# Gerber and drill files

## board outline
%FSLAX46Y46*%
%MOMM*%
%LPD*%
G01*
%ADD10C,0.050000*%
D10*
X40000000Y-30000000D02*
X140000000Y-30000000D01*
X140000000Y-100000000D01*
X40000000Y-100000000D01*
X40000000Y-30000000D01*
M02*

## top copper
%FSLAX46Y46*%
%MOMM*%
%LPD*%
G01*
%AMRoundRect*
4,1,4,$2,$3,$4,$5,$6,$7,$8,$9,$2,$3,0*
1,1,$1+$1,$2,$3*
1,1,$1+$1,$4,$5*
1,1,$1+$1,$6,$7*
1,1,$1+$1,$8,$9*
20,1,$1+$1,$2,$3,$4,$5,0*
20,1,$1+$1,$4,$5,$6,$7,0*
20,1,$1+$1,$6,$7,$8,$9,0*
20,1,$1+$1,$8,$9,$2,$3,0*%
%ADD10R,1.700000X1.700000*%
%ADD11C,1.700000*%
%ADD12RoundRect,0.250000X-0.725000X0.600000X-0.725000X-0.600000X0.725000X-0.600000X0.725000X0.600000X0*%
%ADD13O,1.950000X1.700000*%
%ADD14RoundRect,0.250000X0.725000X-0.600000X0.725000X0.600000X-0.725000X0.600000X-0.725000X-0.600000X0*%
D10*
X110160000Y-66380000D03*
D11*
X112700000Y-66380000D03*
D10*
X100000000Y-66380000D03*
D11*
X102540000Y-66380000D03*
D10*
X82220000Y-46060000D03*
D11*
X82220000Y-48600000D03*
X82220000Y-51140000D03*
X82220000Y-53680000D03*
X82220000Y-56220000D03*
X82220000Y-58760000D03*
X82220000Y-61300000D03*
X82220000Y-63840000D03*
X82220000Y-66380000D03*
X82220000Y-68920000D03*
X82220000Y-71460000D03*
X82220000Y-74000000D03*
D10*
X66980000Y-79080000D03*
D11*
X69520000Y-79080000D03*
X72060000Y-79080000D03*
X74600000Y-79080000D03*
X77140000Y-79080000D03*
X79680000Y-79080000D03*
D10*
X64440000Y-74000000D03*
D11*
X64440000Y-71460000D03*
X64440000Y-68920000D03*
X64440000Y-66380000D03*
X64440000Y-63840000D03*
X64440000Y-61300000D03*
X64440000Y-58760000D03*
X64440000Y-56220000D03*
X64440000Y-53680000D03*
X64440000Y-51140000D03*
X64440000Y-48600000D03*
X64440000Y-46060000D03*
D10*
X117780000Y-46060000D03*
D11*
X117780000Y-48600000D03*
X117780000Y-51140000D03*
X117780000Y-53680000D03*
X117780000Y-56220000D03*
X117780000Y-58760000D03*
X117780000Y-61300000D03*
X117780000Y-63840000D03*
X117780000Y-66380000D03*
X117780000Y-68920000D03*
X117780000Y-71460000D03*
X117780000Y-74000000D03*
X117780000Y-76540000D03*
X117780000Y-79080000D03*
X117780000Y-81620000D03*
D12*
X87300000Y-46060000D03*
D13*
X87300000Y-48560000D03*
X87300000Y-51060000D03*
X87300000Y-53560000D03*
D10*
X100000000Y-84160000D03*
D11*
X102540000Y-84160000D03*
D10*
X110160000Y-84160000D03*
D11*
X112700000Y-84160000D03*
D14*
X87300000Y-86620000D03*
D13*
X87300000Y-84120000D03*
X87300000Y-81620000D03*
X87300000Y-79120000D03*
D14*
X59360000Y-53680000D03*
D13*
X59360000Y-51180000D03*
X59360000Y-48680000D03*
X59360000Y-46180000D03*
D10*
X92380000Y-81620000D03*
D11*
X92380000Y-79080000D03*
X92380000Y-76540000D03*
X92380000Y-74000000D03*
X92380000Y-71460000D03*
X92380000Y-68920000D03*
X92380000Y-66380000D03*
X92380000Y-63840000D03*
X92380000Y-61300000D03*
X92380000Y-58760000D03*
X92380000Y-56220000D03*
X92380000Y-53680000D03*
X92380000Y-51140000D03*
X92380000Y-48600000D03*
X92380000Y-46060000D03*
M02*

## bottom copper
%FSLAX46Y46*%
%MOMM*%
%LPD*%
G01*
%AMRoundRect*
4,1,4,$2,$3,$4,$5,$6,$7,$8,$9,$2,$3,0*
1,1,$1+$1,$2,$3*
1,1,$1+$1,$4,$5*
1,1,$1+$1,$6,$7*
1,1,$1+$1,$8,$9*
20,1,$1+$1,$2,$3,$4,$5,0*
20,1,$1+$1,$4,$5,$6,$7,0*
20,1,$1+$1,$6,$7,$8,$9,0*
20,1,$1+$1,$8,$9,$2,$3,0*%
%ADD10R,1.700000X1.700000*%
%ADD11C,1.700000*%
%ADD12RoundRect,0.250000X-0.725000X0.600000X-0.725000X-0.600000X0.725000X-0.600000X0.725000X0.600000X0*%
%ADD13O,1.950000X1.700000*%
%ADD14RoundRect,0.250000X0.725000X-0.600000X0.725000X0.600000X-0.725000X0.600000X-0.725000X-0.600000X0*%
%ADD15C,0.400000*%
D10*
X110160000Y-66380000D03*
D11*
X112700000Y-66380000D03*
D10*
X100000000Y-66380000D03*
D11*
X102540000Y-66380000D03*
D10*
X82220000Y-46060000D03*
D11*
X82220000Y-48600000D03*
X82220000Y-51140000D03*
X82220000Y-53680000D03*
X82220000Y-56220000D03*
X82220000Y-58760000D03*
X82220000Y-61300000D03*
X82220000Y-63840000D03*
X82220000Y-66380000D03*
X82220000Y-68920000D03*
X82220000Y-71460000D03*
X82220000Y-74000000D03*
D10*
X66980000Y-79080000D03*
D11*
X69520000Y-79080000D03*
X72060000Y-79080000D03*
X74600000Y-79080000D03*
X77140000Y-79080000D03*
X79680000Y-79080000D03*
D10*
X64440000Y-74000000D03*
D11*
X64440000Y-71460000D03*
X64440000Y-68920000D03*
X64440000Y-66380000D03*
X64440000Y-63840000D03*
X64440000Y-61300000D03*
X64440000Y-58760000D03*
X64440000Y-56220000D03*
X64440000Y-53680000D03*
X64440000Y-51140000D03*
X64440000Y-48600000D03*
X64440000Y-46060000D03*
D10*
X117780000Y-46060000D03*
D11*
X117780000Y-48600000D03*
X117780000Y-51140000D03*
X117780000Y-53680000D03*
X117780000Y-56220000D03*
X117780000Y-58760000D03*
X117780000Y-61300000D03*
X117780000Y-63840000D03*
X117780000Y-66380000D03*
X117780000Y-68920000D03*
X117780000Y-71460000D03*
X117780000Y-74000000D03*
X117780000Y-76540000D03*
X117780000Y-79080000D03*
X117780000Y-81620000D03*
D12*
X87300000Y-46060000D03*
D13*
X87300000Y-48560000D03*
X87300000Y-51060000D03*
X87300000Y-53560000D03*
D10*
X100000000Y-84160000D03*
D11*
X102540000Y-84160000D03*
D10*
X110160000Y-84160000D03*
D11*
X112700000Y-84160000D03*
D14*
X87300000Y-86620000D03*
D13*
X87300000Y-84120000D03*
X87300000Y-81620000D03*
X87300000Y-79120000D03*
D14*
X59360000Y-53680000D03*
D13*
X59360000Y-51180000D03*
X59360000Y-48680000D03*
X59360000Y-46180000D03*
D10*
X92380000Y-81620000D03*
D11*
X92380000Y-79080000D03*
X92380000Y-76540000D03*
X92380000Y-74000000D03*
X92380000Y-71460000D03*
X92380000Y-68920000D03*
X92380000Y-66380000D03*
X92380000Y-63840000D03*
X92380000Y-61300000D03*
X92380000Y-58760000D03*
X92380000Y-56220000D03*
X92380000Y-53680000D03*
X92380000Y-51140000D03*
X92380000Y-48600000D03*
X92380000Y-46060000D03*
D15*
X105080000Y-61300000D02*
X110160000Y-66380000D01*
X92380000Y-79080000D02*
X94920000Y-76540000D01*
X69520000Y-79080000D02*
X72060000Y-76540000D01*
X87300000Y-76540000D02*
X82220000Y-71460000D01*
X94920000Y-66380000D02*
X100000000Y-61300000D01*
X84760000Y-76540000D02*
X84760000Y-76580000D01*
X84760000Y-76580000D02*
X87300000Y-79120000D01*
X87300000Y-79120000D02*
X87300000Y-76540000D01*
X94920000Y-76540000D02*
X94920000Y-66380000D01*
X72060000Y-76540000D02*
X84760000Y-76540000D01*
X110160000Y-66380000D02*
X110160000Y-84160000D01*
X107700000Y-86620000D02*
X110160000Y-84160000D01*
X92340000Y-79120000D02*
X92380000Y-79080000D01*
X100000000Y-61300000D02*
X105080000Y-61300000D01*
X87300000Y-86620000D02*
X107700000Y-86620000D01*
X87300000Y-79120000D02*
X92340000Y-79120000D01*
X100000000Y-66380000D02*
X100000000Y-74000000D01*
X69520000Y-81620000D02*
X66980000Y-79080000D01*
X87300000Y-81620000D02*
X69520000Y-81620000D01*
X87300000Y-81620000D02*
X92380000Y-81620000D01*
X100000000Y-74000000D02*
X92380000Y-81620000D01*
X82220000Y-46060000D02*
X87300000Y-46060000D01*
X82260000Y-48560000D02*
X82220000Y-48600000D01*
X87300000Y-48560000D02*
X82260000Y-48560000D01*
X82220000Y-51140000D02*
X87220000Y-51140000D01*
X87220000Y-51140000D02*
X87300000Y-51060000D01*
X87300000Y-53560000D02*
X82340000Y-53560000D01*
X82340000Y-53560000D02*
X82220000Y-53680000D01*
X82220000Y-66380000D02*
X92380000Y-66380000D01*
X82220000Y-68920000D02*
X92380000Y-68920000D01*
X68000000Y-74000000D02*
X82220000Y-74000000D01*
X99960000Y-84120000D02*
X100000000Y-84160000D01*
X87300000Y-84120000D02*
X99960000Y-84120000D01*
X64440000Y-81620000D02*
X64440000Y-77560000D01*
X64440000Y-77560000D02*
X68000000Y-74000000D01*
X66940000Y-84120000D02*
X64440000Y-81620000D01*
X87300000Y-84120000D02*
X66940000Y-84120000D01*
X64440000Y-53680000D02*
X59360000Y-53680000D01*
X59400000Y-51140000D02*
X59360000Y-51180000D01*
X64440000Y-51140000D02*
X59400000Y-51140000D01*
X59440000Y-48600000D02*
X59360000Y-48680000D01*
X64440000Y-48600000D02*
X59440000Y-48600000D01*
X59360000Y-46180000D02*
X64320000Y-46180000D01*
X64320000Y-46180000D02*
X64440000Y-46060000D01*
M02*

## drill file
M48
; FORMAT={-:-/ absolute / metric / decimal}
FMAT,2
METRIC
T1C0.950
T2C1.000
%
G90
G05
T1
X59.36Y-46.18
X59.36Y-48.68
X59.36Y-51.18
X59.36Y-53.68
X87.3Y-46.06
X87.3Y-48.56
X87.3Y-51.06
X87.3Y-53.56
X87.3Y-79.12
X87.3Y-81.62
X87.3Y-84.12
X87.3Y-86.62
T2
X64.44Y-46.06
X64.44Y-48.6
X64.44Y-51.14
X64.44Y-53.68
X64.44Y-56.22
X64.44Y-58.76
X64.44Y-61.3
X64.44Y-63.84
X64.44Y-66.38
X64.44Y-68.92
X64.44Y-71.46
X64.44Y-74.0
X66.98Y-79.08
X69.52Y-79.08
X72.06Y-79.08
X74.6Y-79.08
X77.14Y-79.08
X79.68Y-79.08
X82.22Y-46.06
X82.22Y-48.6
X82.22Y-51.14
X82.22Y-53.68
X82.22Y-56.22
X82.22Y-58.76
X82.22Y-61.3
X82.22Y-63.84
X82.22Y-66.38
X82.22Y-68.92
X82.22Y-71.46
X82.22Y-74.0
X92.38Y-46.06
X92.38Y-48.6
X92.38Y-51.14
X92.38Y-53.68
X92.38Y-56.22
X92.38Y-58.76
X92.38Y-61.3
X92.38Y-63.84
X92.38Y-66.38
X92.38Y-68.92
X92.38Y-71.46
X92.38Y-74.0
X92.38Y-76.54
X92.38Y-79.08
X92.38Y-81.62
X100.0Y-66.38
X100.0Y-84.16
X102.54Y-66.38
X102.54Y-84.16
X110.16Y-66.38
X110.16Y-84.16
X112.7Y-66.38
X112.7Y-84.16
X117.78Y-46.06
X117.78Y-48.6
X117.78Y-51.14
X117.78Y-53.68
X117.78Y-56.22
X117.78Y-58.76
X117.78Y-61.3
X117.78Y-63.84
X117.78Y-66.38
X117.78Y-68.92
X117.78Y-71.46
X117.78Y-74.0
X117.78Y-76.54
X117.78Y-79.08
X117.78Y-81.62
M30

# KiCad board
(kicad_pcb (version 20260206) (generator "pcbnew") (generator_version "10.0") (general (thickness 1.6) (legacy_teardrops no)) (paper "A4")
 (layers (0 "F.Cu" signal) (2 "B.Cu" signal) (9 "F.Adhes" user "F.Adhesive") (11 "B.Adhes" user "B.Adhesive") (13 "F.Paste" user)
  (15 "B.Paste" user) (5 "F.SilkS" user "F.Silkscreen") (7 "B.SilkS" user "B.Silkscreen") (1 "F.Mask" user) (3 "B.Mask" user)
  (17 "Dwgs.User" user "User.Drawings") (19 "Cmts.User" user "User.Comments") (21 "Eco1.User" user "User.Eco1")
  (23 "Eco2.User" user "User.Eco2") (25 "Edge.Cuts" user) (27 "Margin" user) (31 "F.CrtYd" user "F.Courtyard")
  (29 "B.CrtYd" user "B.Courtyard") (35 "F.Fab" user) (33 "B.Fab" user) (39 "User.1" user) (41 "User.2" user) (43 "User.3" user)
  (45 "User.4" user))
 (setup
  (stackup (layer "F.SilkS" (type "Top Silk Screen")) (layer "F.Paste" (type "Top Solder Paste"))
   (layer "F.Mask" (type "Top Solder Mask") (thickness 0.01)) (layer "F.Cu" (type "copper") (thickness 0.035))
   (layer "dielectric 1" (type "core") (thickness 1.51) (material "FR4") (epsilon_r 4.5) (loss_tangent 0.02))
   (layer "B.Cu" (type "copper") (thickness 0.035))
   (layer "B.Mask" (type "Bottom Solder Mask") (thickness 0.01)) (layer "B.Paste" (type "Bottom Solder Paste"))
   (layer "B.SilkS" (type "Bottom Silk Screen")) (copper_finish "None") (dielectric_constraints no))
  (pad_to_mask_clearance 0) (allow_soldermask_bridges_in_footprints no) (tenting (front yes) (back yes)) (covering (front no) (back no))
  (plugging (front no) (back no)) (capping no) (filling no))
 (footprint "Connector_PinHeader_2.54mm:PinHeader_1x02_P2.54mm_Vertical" (layer "F.Cu") (at 110.16 66.38 90)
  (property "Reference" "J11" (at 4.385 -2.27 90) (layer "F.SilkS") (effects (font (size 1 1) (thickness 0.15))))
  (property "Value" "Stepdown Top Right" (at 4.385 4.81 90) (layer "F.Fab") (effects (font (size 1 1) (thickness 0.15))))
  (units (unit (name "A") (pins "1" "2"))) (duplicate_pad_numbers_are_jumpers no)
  (pad "1" thru_hole rect (at 0 0 90) (size 1.7 1.7) (drill 1) (layers "*.Cu" "*.Mask") (remove_unused_layers no) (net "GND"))
  (pad "2" thru_hole circle (at 0 2.54 90) (size 1.7 1.7) (drill 1) (layers "*.Cu" "*.Mask") (remove_unused_layers no) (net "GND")))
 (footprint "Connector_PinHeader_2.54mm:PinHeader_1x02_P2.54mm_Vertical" (layer "F.Cu") (at 100 66.38 90)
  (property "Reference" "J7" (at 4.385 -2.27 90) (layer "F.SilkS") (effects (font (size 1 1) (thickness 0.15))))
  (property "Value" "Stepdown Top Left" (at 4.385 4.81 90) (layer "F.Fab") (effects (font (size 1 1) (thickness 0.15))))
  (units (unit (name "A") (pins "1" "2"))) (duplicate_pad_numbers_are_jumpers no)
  (pad "1" thru_hole rect (at 0 0 90) (size 1.7 1.7) (drill 1) (layers "*.Cu" "*.Mask") (remove_unused_layers no) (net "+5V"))
  (pad "2" thru_hole circle (at 0 2.54 90) (size 1.7 1.7) (drill 1) (layers "*.Cu" "*.Mask") (remove_unused_layers no) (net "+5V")))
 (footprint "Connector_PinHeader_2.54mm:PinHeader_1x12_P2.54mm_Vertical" (layer "F.Cu") (at 82.22 46.06)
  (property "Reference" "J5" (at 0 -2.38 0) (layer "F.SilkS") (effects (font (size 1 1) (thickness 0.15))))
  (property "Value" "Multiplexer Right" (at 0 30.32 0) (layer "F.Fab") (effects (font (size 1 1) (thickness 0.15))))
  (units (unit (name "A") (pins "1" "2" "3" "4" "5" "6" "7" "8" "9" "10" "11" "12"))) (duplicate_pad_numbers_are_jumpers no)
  (pad "1" thru_hole rect (at 0 0) (size 1.7 1.7) (drill 1) (layers "*.Cu" "*.Mask") (remove_unused_layers no) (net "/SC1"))
  (pad "2" thru_hole circle (at 0 2.54) (size 1.7 1.7) (drill 1) (layers "*.Cu" "*.Mask") (remove_unused_layers no) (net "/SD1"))
  (pad "3" thru_hole circle (at 0 5.08) (size 1.7 1.7) (drill 1) (layers "*.Cu" "*.Mask") (remove_unused_layers no) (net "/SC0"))
  (pad "4" thru_hole circle (at 0 7.62) (size 1.7 1.7) (drill 1) (layers "*.Cu" "*.Mask") (remove_unused_layers no) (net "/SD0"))
  (pad "5" thru_hole circle (at 0 10.16) (size 1.7 1.7) (drill 1) (layers "*.Cu" "*.Mask") (remove_unused_layers no)
   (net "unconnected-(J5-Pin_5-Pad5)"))
  (pad "6" thru_hole circle (at 0 12.7) (size 1.7 1.7) (drill 1) (layers "*.Cu" "*.Mask") (remove_unused_layers no)
   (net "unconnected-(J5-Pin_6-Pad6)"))
  (pad "7" thru_hole circle (at 0 15.24) (size 1.7 1.7) (drill 1) (layers "*.Cu" "*.Mask") (remove_unused_layers no)
   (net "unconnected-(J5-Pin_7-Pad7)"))
  (pad "8" thru_hole circle (at 0 17.78) (size 1.7 1.7) (drill 1) (layers "*.Cu" "*.Mask") (remove_unused_layers no)
   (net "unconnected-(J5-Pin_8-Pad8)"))
  (pad "9" thru_hole circle (at 0 20.32) (size 1.7 1.7) (drill 1) (layers "*.Cu" "*.Mask") (remove_unused_layers no) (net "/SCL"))
  (pad "10" thru_hole circle (at 0 22.86) (size 1.7 1.7) (drill 1) (layers "*.Cu" "*.Mask") (remove_unused_layers no) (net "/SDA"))
  (pad "11" thru_hole circle (at 0 25.4) (size 1.7 1.7) (drill 1) (layers "*.Cu" "*.Mask") (remove_unused_layers no) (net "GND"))
  (pad "12" thru_hole circle (at 0 27.94) (size 1.7 1.7) (drill 1) (layers "*.Cu" "*.Mask") (remove_unused_layers no) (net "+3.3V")))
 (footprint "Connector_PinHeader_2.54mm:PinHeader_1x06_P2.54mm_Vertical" (layer "F.Cu") (at 66.98 79.08 90)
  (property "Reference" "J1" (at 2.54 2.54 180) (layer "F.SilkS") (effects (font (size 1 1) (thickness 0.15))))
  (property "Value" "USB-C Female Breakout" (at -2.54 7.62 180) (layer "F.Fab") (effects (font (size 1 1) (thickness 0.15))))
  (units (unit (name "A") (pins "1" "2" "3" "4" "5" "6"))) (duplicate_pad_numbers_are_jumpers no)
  (pad "1" thru_hole rect (at 0 0 90) (size 1.7 1.7) (drill 1) (layers "*.Cu" "*.Mask") (remove_unused_layers no) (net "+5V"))
  (pad "2" thru_hole circle (at 0 2.54 90) (size 1.7 1.7) (drill 1) (layers "*.Cu" "*.Mask") (remove_unused_layers no) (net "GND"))
  (pad "3" thru_hole circle (at 0 5.08 90) (size 1.7 1.7) (drill 1) (layers "*.Cu" "*.Mask") (remove_unused_layers no)
   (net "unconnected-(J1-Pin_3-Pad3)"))
  (pad "4" thru_hole circle (at 0 7.62 90) (size 1.7 1.7) (drill 1) (layers "*.Cu" "*.Mask") (remove_unused_layers no)
   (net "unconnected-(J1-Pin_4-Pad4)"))
  (pad "5" thru_hole circle (at 0 10.16 90) (size 1.7 1.7) (drill 1) (layers "*.Cu" "*.Mask") (remove_unused_layers no)
   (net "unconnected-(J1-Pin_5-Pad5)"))
  (pad "6" thru_hole circle (at 0 12.7 90) (size 1.7 1.7) (drill 1) (layers "*.Cu" "*.Mask") (remove_unused_layers no)
   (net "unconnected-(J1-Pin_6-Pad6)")))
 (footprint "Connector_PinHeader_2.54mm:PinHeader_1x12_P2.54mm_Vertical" (layer "F.Cu") (at 64.44 74 180)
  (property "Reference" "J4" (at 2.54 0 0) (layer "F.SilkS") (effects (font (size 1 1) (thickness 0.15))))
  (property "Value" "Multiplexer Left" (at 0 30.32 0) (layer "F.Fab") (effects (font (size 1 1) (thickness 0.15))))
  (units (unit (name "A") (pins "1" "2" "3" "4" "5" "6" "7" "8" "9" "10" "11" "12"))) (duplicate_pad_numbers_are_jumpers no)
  (pad "1" thru_hole rect (at 0 0 180) (size 1.7 1.7) (drill 1) (layers "*.Cu" "*.Mask") (remove_unused_layers no)
   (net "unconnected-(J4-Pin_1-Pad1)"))
  (pad "2" thru_hole circle (at 0 2.54 180) (size 1.7 1.7) (drill 1) (layers "*.Cu" "*.Mask") (remove_unused_layers no)
   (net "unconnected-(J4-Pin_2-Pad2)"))
  (pad "3" thru_hole circle (at 0 5.08 180) (size 1.7 1.7) (drill 1) (layers "*.Cu" "*.Mask") (remove_unused_layers no)
   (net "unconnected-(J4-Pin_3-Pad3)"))
  (pad "4" thru_hole circle (at 0 7.62 180) (size 1.7 1.7) (drill 1) (layers "*.Cu" "*.Mask") (remove_unused_layers no)
   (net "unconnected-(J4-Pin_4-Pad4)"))
  (pad "5" thru_hole circle (at 0 10.16 180) (size 1.7 1.7) (drill 1) (layers "*.Cu" "*.Mask") (remove_unused_layers no)
   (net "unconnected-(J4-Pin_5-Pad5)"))
  (pad "6" thru_hole circle (at 0 12.7 180) (size 1.7 1.7) (drill 1) (layers "*.Cu" "*.Mask") (remove_unused_layers no)
   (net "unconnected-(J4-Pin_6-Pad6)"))
  (pad "7" thru_hole circle (at 0 15.24 180) (size 1.7 1.7) (drill 1) (layers "*.Cu" "*.Mask") (remove_unused_layers no)
   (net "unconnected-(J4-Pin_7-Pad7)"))
  (pad "8" thru_hole circle (at 0 17.78 180) (size 1.7 1.7) (drill 1) (layers "*.Cu" "*.Mask") (remove_unused_layers no)
   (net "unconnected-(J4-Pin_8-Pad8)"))
  (pad "9" thru_hole circle (at 0 20.32 180) (size 1.7 1.7) (drill 1) (layers "*.Cu" "*.Mask") (remove_unused_layers no) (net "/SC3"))
  (pad "10" thru_hole circle (at 0 22.86 180) (size 1.7 1.7) (drill 1) (layers "*.Cu" "*.Mask") (remove_unused_layers no) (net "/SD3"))
  (pad "11" thru_hole circle (at 0 25.4 180) (size 1.7 1.7) (drill 1) (layers "*.Cu" "*.Mask") (remove_unused_layers no) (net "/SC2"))
  (pad "12" thru_hole circle (at 0 27.94 180) (size 1.7 1.7) (drill 1) (layers "*.Cu" "*.Mask") (remove_unused_layers no) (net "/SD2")))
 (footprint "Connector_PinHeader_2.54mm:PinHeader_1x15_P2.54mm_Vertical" (layer "F.Cu") (at 117.78 46.06)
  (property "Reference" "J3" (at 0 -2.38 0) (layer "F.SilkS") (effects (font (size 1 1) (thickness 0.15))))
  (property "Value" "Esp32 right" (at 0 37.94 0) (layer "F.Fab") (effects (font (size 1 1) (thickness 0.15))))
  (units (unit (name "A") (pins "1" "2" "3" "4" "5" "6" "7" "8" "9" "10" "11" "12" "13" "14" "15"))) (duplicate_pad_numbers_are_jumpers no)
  (pad "1" thru_hole rect (at 0 0) (size 1.7 1.7) (drill 1) (layers "*.Cu" "*.Mask") (remove_unused_layers no)
   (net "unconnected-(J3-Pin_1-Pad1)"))
  (pad "2" thru_hole circle (at 0 2.54) (size 1.7 1.7) (drill 1) (layers "*.Cu" "*.Mask") (remove_unused_layers no)
   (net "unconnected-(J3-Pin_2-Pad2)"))
  (pad "3" thru_hole circle (at 0 5.08) (size 1.7 1.7) (drill 1) (layers "*.Cu" "*.Mask") (remove_unused_layers no)
   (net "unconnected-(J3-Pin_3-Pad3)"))
  (pad "4" thru_hole circle (at 0 7.62) (size 1.7 1.7) (drill 1) (layers "*.Cu" "*.Mask") (remove_unused_layers no)
   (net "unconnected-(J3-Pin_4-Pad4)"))
  (pad "5" thru_hole circle (at 0 10.16) (size 1.7 1.7) (drill 1) (layers "*.Cu" "*.Mask") (remove_unused_layers no)
   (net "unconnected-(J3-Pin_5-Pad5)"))
  (pad "6" thru_hole circle (at 0 12.7) (size 1.7 1.7) (drill 1) (layers "*.Cu" "*.Mask") (remove_unused_layers no)
   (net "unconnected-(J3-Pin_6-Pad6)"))
  (pad "7" thru_hole circle (at 0 15.24) (size 1.7 1.7) (drill 1) (layers "*.Cu" "*.Mask") (remove_unused_layers no)
   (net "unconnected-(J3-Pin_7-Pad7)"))
  (pad "8" thru_hole circle (at 0 17.78) (size 1.7 1.7) (drill 1) (layers "*.Cu" "*.Mask") (remove_unused_layers no)
   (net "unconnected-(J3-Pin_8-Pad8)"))
  (pad "9" thru_hole circle (at 0 20.32) (size 1.7 1.7) (drill 1) (layers "*.Cu" "*.Mask") (remove_unused_layers no)
   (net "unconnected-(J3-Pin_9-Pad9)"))
  (pad "10" thru_hole circle (at 0 22.86) (size 1.7 1.7) (drill 1) (layers "*.Cu" "*.Mask") (remove_unused_layers no)
   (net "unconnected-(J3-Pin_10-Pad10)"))
  (pad "11" thru_hole circle (at 0 25.4) (size 1.7 1.7) (drill 1) (layers "*.Cu" "*.Mask") (remove_unused_layers no)
   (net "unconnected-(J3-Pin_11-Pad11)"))
  (pad "12" thru_hole circle (at 0 27.94) (size 1.7 1.7) (drill 1) (layers "*.Cu" "*.Mask") (remove_unused_layers no)
   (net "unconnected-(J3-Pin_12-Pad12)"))
  (pad "13" thru_hole circle (at 0 30.48) (size 1.7 1.7) (drill 1) (layers "*.Cu" "*.Mask") (remove_unused_layers no)
   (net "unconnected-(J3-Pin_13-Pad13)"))
  (pad "14" thru_hole circle (at 0 33.02) (size 1.7 1.7) (drill 1) (layers "*.Cu" "*.Mask") (remove_unused_layers no)
   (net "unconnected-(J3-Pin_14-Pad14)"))
  (pad "15" thru_hole circle (at 0 35.56) (size 1.7 1.7) (drill 1) (layers "*.Cu" "*.Mask") (remove_unused_layers no)
   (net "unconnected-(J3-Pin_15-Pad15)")))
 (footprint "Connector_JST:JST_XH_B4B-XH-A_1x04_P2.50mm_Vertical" (layer "F.Cu") (at 87.3 46.06 -90)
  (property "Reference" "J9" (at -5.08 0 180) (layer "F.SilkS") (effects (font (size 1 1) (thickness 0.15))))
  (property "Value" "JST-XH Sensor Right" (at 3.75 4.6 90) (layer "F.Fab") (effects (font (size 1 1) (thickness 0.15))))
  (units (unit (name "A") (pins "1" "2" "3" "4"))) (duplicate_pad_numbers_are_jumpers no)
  (pad "1" thru_hole roundrect (at 0 0 270) (size 1.7 1.95) (drill 0.95) (layers "*.Cu" "*.Mask") (remove_unused_layers no)
   (roundrect_rratio 0.147059) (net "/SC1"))
  (pad "2" thru_hole oval (at 2.5 0 270) (size 1.7 1.95) (drill 0.95) (layers "*.Cu" "*.Mask") (remove_unused_layers no) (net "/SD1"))
  (pad "3" thru_hole oval (at 5 0 270) (size 1.7 1.95) (drill 0.95) (layers "*.Cu" "*.Mask") (remove_unused_layers no) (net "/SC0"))
  (pad "4" thru_hole oval (at 7.5 0 270) (size 1.7 1.95) (drill 0.95) (layers "*.Cu" "*.Mask") (remove_unused_layers no) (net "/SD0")))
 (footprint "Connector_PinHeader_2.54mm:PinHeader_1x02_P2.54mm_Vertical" (layer "F.Cu") (at 100 84.16 90)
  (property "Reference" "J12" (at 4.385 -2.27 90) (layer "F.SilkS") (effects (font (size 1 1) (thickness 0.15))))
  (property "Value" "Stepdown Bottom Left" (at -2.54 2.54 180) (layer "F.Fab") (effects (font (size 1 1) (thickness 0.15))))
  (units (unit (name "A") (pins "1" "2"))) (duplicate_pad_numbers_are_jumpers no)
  (pad "1" thru_hole rect (at 0 0 90) (size 1.7 1.7) (drill 1) (layers "*.Cu" "*.Mask") (remove_unused_layers no) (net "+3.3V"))
  (pad "2" thru_hole circle (at 0 2.54 90) (size 1.7 1.7) (drill 1) (layers "*.Cu" "*.Mask") (remove_unused_layers no) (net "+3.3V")))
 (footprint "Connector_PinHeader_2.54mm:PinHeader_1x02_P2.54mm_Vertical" (layer "F.Cu") (at 110.16 84.16 90)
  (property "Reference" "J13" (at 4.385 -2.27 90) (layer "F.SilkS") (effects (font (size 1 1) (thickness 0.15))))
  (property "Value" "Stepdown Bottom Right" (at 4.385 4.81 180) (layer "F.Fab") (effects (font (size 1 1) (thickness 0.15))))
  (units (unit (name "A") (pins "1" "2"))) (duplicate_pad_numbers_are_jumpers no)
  (pad "1" thru_hole rect (at 0 0 90) (size 1.7 1.7) (drill 1) (layers "*.Cu" "*.Mask") (remove_unused_layers no) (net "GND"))
  (pad "2" thru_hole circle (at 0 2.54 90) (size 1.7 1.7) (drill 1) (layers "*.Cu" "*.Mask") (remove_unused_layers no) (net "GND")))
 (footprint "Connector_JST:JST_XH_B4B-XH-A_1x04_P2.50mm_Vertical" (layer "F.Cu") (at 87.3 86.62 90)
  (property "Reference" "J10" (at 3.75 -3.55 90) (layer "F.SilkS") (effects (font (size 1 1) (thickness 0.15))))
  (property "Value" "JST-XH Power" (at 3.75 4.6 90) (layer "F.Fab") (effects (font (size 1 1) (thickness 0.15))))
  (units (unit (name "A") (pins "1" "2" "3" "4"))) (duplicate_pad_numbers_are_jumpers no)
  (pad "1" thru_hole roundrect (at 0 0 90) (size 1.7 1.95) (drill 0.95) (layers "*.Cu" "*.Mask") (remove_unused_layers no)
   (roundrect_rratio 0.147059) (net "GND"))
  (pad "2" thru_hole oval (at 2.5 0 90) (size 1.7 1.95) (drill 0.95) (layers "*.Cu" "*.Mask") (remove_unused_layers no) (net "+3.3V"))
  (pad "3" thru_hole oval (at 5 0 90) (size 1.7 1.95) (drill 0.95) (layers "*.Cu" "*.Mask") (remove_unused_layers no) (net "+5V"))
  (pad "4" thru_hole oval (at 7.5 0 90) (size 1.7 1.95) (drill 0.95) (layers "*.Cu" "*.Mask") (remove_unused_layers no) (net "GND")))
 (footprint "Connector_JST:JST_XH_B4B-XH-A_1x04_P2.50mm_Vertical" (layer "F.Cu") (at 59.36 53.68 90)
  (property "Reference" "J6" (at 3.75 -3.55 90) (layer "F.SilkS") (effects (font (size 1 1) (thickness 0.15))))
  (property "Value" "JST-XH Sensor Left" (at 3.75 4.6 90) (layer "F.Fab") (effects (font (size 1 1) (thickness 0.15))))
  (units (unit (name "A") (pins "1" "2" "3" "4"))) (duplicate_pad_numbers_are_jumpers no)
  (pad "1" thru_hole roundrect (at 0 0 90) (size 1.7 1.95) (drill 0.95) (layers "*.Cu" "*.Mask") (remove_unused_layers no)
   (roundrect_rratio 0.147059) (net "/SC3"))
  (pad "2" thru_hole oval (at 2.5 0 90) (size 1.7 1.95) (drill 0.95) (layers "*.Cu" "*.Mask") (remove_unused_layers no) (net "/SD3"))
  (pad "3" thru_hole oval (at 5 0 90) (size 1.7 1.95) (drill 0.95) (layers "*.Cu" "*.Mask") (remove_unused_layers no) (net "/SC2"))
  (pad "4" thru_hole oval (at 7.5 0 90) (size 1.7 1.95) (drill 0.95) (layers "*.Cu" "*.Mask") (remove_unused_layers no) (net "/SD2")))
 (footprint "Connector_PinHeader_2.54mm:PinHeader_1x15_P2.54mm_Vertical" (layer "F.Cu") (at 92.38 81.62 180)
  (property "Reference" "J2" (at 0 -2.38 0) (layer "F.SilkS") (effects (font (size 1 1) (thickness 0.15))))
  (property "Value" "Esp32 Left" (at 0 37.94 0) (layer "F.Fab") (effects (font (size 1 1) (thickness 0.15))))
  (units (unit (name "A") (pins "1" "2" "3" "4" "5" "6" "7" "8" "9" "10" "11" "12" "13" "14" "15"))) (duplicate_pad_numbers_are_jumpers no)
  (pad "1" thru_hole rect (at 0 0 180) (size 1.7 1.7) (drill 1) (layers "*.Cu" "*.Mask") (remove_unused_layers no) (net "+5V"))
  (pad "2" thru_hole circle (at 0 2.54 180) (size 1.7 1.7) (drill 1) (layers "*.Cu" "*.Mask") (remove_unused_layers no) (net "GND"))
  (pad "3" thru_hole circle (at 0 5.08 180) (size 1.7 1.7) (drill 1) (layers "*.Cu" "*.Mask") (remove_unused_layers no)
   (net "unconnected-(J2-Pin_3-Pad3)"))
  (pad "4" thru_hole circle (at 0 7.62 180) (size 1.7 1.7) (drill 1) (layers "*.Cu" "*.Mask") (remove_unused_layers no)
   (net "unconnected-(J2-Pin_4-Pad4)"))
  (pad "5" thru_hole circle (at 0 10.16 180) (size 1.7 1.7) (drill 1) (layers "*.Cu" "*.Mask") (remove_unused_layers no)
   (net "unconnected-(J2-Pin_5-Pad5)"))
  (pad "6" thru_hole circle (at 0 12.7 180) (size 1.7 1.7) (drill 1) (layers "*.Cu" "*.Mask") (remove_unused_layers no) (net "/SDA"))
  (pad "7" thru_hole circle (at 0 15.24 180) (size 1.7 1.7) (drill 1) (layers "*.Cu" "*.Mask") (remove_unused_layers no) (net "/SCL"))
  (pad "8" thru_hole circle (at 0 17.78 180) (size 1.7 1.7) (drill 1) (layers "*.Cu" "*.Mask") (remove_unused_layers no)
   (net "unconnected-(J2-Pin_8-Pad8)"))
  (pad "9" thru_hole circle (at 0 20.32 180) (size 1.7 1.7) (drill 1) (layers "*.Cu" "*.Mask") (remove_unused_layers no)
   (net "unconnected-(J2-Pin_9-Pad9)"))
  (pad "10" thru_hole circle (at 0 22.86 180) (size 1.7 1.7) (drill 1) (layers "*.Cu" "*.Mask") (remove_unused_layers no)
   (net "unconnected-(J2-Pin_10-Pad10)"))
  (pad "11" thru_hole circle (at 0 25.4 180) (size 1.7 1.7) (drill 1) (layers "*.Cu" "*.Mask") (remove_unused_layers no)
   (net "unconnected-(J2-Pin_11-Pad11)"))
  (pad "12" thru_hole circle (at 0 27.94 180) (size 1.7 1.7) (drill 1) (layers "*.Cu" "*.Mask") (remove_unused_layers no)
   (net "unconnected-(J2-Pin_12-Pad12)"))
  (pad "13" thru_hole circle (at 0 30.48 180) (size 1.7 1.7) (drill 1) (layers "*.Cu" "*.Mask") (remove_unused_layers no)
   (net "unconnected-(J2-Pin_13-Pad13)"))
  (pad "14" thru_hole circle (at 0 33.02 180) (size 1.7 1.7) (drill 1) (layers "*.Cu" "*.Mask") (remove_unused_layers no)
   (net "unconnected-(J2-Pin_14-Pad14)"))
  (pad "15" thru_hole circle (at 0 35.56 180) (size 1.7 1.7) (drill 1) (layers "*.Cu" "*.Mask") (remove_unused_layers no)
   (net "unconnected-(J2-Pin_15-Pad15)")))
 (gr_rect (start 40 30) (end 140 100) (stroke (width 0.05) (type default)) (fill no) (layer "Edge.Cuts"))
 (segment (start 105.08 61.3) (end 110.16 66.38) (width 0.4) (layer "B.Cu") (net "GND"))
 (segment (start 92.38 79.08) (end 94.92 76.54) (width 0.4) (layer "B.Cu") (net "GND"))
 (segment (start 69.52 79.08) (end 72.06 76.54) (width 0.4) (layer "B.Cu") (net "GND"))
 (segment (start 87.3 76.54) (end 82.22 71.46) (width 0.4) (layer "B.Cu") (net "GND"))
 (segment (start 94.92 66.38) (end 100 61.3) (width 0.4) (layer "B.Cu") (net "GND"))
 (segment (start 84.76 76.54) (end 84.76 76.58) (width 0.4) (layer "B.Cu") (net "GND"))
 (segment (start 84.76 76.58) (end 87.3 79.12) (width 0.4) (layer "B.Cu") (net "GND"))
 (segment (start 87.3 79.12) (end 87.3 76.54) (width 0.4) (layer "B.Cu") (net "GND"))
 (segment (start 94.92 76.54) (end 94.92 66.38) (width 0.4) (layer "B.Cu") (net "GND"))
 (segment (start 72.06 76.54) (end 84.76 76.54) (width 0.4) (layer "B.Cu") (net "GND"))
 (segment (start 110.16 66.38) (end 110.16 84.16) (width 0.4) (layer "B.Cu") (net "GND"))
 (segment (start 107.7 86.62) (end 110.16 84.16) (width 0.4) (layer "B.Cu") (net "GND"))
 (segment (start 92.34 79.12) (end 92.38 79.08) (width 0.4) (layer "B.Cu") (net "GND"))
 (segment (start 100 61.3) (end 105.08 61.3) (width 0.4) (layer "B.Cu") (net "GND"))
 (segment (start 87.3 86.62) (end 107.7 86.62) (width 0.4) (layer "B.Cu") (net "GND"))
 (segment (start 87.3 79.12) (end 92.34 79.12) (width 0.4) (layer "B.Cu") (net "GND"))
 (segment (start 100 66.38) (end 100 74) (width 0.4) (layer "B.Cu") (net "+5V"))
 (segment (start 69.52 81.62) (end 66.98 79.08) (width 0.4) (layer "B.Cu") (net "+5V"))
 (segment (start 87.3 81.62) (end 69.52 81.62) (width 0.4) (layer "B.Cu") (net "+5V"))
 (segment (start 87.3 81.62) (end 92.38 81.62) (width 0.4) (layer "B.Cu") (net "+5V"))
 (segment (start 100 74) (end 92.38 81.62) (width 0.4) (layer "B.Cu") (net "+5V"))
 (segment (start 82.22 46.06) (end 87.3 46.06) (width 0.4) (layer "B.Cu") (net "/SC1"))
 (segment (start 82.26 48.56) (end 82.22 48.6) (width 0.4) (layer "B.Cu") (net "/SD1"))
 (segment (start 87.3 48.56) (end 82.26 48.56) (width 0.4) (layer "B.Cu") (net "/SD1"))
 (segment (start 82.22 51.14) (end 87.22 51.14) (width 0.4) (layer "B.Cu") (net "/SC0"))
 (segment (start 87.22 51.14) (end 87.3 51.06) (width 0.4) (layer "B.Cu") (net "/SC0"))
 (segment (start 87.3 53.56) (end 82.34 53.56) (width 0.4) (layer "B.Cu") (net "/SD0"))
 (segment (start 82.34 53.56) (end 82.22 53.68) (width 0.4) (layer "B.Cu") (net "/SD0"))
 (segment (start 82.22 66.38) (end 92.38 66.38) (width 0.4) (layer "B.Cu") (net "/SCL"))
 (segment (start 82.22 68.92) (end 92.38 68.92) (width 0.4) (layer "B.Cu") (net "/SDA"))
 (segment (start 68 74) (end 82.22 74) (width 0.4) (layer "B.Cu") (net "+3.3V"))
 (segment (start 99.96 84.12) (end 100 84.16) (width 0.4) (layer "B.Cu") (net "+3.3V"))
 (segment (start 87.3 84.12) (end 99.96 84.12) (width 0.4) (layer "B.Cu") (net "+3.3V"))
 (segment (start 64.44 81.62) (end 64.44 77.56) (width 0.4) (layer "B.Cu") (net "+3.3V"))
 (segment (start 64.44 77.56) (end 68 74) (width 0.4) (layer "B.Cu") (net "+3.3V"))
 (segment (start 66.94 84.12) (end 64.44 81.62) (width 0.4) (layer "B.Cu") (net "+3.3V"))
 (segment (start 87.3 84.12) (end 66.94 84.12) (width 0.4) (layer "B.Cu") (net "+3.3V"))
 (segment (start 64.44 53.68) (end 59.36 53.68) (width 0.4) (layer "B.Cu") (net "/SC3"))
 (segment (start 59.4 51.14) (end 59.36 51.18) (width 0.4) (layer "B.Cu") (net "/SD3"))
 (segment (start 64.44 51.14) (end 59.4 51.14) (width 0.4) (layer "B.Cu") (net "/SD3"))
 (segment (start 59.44 48.6) (end 59.36 48.68) (width 0.4) (layer "B.Cu") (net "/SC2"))
 (segment (start 64.44 48.6) (end 59.44 48.6) (width 0.4) (layer "B.Cu") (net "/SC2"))
 (segment (start 59.36 46.18) (end 64.32 46.18) (width 0.4) (layer "B.Cu") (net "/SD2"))
 (segment (start 64.32 46.18) (end 64.44 46.06) (width 0.4) (layer "B.Cu") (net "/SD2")))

